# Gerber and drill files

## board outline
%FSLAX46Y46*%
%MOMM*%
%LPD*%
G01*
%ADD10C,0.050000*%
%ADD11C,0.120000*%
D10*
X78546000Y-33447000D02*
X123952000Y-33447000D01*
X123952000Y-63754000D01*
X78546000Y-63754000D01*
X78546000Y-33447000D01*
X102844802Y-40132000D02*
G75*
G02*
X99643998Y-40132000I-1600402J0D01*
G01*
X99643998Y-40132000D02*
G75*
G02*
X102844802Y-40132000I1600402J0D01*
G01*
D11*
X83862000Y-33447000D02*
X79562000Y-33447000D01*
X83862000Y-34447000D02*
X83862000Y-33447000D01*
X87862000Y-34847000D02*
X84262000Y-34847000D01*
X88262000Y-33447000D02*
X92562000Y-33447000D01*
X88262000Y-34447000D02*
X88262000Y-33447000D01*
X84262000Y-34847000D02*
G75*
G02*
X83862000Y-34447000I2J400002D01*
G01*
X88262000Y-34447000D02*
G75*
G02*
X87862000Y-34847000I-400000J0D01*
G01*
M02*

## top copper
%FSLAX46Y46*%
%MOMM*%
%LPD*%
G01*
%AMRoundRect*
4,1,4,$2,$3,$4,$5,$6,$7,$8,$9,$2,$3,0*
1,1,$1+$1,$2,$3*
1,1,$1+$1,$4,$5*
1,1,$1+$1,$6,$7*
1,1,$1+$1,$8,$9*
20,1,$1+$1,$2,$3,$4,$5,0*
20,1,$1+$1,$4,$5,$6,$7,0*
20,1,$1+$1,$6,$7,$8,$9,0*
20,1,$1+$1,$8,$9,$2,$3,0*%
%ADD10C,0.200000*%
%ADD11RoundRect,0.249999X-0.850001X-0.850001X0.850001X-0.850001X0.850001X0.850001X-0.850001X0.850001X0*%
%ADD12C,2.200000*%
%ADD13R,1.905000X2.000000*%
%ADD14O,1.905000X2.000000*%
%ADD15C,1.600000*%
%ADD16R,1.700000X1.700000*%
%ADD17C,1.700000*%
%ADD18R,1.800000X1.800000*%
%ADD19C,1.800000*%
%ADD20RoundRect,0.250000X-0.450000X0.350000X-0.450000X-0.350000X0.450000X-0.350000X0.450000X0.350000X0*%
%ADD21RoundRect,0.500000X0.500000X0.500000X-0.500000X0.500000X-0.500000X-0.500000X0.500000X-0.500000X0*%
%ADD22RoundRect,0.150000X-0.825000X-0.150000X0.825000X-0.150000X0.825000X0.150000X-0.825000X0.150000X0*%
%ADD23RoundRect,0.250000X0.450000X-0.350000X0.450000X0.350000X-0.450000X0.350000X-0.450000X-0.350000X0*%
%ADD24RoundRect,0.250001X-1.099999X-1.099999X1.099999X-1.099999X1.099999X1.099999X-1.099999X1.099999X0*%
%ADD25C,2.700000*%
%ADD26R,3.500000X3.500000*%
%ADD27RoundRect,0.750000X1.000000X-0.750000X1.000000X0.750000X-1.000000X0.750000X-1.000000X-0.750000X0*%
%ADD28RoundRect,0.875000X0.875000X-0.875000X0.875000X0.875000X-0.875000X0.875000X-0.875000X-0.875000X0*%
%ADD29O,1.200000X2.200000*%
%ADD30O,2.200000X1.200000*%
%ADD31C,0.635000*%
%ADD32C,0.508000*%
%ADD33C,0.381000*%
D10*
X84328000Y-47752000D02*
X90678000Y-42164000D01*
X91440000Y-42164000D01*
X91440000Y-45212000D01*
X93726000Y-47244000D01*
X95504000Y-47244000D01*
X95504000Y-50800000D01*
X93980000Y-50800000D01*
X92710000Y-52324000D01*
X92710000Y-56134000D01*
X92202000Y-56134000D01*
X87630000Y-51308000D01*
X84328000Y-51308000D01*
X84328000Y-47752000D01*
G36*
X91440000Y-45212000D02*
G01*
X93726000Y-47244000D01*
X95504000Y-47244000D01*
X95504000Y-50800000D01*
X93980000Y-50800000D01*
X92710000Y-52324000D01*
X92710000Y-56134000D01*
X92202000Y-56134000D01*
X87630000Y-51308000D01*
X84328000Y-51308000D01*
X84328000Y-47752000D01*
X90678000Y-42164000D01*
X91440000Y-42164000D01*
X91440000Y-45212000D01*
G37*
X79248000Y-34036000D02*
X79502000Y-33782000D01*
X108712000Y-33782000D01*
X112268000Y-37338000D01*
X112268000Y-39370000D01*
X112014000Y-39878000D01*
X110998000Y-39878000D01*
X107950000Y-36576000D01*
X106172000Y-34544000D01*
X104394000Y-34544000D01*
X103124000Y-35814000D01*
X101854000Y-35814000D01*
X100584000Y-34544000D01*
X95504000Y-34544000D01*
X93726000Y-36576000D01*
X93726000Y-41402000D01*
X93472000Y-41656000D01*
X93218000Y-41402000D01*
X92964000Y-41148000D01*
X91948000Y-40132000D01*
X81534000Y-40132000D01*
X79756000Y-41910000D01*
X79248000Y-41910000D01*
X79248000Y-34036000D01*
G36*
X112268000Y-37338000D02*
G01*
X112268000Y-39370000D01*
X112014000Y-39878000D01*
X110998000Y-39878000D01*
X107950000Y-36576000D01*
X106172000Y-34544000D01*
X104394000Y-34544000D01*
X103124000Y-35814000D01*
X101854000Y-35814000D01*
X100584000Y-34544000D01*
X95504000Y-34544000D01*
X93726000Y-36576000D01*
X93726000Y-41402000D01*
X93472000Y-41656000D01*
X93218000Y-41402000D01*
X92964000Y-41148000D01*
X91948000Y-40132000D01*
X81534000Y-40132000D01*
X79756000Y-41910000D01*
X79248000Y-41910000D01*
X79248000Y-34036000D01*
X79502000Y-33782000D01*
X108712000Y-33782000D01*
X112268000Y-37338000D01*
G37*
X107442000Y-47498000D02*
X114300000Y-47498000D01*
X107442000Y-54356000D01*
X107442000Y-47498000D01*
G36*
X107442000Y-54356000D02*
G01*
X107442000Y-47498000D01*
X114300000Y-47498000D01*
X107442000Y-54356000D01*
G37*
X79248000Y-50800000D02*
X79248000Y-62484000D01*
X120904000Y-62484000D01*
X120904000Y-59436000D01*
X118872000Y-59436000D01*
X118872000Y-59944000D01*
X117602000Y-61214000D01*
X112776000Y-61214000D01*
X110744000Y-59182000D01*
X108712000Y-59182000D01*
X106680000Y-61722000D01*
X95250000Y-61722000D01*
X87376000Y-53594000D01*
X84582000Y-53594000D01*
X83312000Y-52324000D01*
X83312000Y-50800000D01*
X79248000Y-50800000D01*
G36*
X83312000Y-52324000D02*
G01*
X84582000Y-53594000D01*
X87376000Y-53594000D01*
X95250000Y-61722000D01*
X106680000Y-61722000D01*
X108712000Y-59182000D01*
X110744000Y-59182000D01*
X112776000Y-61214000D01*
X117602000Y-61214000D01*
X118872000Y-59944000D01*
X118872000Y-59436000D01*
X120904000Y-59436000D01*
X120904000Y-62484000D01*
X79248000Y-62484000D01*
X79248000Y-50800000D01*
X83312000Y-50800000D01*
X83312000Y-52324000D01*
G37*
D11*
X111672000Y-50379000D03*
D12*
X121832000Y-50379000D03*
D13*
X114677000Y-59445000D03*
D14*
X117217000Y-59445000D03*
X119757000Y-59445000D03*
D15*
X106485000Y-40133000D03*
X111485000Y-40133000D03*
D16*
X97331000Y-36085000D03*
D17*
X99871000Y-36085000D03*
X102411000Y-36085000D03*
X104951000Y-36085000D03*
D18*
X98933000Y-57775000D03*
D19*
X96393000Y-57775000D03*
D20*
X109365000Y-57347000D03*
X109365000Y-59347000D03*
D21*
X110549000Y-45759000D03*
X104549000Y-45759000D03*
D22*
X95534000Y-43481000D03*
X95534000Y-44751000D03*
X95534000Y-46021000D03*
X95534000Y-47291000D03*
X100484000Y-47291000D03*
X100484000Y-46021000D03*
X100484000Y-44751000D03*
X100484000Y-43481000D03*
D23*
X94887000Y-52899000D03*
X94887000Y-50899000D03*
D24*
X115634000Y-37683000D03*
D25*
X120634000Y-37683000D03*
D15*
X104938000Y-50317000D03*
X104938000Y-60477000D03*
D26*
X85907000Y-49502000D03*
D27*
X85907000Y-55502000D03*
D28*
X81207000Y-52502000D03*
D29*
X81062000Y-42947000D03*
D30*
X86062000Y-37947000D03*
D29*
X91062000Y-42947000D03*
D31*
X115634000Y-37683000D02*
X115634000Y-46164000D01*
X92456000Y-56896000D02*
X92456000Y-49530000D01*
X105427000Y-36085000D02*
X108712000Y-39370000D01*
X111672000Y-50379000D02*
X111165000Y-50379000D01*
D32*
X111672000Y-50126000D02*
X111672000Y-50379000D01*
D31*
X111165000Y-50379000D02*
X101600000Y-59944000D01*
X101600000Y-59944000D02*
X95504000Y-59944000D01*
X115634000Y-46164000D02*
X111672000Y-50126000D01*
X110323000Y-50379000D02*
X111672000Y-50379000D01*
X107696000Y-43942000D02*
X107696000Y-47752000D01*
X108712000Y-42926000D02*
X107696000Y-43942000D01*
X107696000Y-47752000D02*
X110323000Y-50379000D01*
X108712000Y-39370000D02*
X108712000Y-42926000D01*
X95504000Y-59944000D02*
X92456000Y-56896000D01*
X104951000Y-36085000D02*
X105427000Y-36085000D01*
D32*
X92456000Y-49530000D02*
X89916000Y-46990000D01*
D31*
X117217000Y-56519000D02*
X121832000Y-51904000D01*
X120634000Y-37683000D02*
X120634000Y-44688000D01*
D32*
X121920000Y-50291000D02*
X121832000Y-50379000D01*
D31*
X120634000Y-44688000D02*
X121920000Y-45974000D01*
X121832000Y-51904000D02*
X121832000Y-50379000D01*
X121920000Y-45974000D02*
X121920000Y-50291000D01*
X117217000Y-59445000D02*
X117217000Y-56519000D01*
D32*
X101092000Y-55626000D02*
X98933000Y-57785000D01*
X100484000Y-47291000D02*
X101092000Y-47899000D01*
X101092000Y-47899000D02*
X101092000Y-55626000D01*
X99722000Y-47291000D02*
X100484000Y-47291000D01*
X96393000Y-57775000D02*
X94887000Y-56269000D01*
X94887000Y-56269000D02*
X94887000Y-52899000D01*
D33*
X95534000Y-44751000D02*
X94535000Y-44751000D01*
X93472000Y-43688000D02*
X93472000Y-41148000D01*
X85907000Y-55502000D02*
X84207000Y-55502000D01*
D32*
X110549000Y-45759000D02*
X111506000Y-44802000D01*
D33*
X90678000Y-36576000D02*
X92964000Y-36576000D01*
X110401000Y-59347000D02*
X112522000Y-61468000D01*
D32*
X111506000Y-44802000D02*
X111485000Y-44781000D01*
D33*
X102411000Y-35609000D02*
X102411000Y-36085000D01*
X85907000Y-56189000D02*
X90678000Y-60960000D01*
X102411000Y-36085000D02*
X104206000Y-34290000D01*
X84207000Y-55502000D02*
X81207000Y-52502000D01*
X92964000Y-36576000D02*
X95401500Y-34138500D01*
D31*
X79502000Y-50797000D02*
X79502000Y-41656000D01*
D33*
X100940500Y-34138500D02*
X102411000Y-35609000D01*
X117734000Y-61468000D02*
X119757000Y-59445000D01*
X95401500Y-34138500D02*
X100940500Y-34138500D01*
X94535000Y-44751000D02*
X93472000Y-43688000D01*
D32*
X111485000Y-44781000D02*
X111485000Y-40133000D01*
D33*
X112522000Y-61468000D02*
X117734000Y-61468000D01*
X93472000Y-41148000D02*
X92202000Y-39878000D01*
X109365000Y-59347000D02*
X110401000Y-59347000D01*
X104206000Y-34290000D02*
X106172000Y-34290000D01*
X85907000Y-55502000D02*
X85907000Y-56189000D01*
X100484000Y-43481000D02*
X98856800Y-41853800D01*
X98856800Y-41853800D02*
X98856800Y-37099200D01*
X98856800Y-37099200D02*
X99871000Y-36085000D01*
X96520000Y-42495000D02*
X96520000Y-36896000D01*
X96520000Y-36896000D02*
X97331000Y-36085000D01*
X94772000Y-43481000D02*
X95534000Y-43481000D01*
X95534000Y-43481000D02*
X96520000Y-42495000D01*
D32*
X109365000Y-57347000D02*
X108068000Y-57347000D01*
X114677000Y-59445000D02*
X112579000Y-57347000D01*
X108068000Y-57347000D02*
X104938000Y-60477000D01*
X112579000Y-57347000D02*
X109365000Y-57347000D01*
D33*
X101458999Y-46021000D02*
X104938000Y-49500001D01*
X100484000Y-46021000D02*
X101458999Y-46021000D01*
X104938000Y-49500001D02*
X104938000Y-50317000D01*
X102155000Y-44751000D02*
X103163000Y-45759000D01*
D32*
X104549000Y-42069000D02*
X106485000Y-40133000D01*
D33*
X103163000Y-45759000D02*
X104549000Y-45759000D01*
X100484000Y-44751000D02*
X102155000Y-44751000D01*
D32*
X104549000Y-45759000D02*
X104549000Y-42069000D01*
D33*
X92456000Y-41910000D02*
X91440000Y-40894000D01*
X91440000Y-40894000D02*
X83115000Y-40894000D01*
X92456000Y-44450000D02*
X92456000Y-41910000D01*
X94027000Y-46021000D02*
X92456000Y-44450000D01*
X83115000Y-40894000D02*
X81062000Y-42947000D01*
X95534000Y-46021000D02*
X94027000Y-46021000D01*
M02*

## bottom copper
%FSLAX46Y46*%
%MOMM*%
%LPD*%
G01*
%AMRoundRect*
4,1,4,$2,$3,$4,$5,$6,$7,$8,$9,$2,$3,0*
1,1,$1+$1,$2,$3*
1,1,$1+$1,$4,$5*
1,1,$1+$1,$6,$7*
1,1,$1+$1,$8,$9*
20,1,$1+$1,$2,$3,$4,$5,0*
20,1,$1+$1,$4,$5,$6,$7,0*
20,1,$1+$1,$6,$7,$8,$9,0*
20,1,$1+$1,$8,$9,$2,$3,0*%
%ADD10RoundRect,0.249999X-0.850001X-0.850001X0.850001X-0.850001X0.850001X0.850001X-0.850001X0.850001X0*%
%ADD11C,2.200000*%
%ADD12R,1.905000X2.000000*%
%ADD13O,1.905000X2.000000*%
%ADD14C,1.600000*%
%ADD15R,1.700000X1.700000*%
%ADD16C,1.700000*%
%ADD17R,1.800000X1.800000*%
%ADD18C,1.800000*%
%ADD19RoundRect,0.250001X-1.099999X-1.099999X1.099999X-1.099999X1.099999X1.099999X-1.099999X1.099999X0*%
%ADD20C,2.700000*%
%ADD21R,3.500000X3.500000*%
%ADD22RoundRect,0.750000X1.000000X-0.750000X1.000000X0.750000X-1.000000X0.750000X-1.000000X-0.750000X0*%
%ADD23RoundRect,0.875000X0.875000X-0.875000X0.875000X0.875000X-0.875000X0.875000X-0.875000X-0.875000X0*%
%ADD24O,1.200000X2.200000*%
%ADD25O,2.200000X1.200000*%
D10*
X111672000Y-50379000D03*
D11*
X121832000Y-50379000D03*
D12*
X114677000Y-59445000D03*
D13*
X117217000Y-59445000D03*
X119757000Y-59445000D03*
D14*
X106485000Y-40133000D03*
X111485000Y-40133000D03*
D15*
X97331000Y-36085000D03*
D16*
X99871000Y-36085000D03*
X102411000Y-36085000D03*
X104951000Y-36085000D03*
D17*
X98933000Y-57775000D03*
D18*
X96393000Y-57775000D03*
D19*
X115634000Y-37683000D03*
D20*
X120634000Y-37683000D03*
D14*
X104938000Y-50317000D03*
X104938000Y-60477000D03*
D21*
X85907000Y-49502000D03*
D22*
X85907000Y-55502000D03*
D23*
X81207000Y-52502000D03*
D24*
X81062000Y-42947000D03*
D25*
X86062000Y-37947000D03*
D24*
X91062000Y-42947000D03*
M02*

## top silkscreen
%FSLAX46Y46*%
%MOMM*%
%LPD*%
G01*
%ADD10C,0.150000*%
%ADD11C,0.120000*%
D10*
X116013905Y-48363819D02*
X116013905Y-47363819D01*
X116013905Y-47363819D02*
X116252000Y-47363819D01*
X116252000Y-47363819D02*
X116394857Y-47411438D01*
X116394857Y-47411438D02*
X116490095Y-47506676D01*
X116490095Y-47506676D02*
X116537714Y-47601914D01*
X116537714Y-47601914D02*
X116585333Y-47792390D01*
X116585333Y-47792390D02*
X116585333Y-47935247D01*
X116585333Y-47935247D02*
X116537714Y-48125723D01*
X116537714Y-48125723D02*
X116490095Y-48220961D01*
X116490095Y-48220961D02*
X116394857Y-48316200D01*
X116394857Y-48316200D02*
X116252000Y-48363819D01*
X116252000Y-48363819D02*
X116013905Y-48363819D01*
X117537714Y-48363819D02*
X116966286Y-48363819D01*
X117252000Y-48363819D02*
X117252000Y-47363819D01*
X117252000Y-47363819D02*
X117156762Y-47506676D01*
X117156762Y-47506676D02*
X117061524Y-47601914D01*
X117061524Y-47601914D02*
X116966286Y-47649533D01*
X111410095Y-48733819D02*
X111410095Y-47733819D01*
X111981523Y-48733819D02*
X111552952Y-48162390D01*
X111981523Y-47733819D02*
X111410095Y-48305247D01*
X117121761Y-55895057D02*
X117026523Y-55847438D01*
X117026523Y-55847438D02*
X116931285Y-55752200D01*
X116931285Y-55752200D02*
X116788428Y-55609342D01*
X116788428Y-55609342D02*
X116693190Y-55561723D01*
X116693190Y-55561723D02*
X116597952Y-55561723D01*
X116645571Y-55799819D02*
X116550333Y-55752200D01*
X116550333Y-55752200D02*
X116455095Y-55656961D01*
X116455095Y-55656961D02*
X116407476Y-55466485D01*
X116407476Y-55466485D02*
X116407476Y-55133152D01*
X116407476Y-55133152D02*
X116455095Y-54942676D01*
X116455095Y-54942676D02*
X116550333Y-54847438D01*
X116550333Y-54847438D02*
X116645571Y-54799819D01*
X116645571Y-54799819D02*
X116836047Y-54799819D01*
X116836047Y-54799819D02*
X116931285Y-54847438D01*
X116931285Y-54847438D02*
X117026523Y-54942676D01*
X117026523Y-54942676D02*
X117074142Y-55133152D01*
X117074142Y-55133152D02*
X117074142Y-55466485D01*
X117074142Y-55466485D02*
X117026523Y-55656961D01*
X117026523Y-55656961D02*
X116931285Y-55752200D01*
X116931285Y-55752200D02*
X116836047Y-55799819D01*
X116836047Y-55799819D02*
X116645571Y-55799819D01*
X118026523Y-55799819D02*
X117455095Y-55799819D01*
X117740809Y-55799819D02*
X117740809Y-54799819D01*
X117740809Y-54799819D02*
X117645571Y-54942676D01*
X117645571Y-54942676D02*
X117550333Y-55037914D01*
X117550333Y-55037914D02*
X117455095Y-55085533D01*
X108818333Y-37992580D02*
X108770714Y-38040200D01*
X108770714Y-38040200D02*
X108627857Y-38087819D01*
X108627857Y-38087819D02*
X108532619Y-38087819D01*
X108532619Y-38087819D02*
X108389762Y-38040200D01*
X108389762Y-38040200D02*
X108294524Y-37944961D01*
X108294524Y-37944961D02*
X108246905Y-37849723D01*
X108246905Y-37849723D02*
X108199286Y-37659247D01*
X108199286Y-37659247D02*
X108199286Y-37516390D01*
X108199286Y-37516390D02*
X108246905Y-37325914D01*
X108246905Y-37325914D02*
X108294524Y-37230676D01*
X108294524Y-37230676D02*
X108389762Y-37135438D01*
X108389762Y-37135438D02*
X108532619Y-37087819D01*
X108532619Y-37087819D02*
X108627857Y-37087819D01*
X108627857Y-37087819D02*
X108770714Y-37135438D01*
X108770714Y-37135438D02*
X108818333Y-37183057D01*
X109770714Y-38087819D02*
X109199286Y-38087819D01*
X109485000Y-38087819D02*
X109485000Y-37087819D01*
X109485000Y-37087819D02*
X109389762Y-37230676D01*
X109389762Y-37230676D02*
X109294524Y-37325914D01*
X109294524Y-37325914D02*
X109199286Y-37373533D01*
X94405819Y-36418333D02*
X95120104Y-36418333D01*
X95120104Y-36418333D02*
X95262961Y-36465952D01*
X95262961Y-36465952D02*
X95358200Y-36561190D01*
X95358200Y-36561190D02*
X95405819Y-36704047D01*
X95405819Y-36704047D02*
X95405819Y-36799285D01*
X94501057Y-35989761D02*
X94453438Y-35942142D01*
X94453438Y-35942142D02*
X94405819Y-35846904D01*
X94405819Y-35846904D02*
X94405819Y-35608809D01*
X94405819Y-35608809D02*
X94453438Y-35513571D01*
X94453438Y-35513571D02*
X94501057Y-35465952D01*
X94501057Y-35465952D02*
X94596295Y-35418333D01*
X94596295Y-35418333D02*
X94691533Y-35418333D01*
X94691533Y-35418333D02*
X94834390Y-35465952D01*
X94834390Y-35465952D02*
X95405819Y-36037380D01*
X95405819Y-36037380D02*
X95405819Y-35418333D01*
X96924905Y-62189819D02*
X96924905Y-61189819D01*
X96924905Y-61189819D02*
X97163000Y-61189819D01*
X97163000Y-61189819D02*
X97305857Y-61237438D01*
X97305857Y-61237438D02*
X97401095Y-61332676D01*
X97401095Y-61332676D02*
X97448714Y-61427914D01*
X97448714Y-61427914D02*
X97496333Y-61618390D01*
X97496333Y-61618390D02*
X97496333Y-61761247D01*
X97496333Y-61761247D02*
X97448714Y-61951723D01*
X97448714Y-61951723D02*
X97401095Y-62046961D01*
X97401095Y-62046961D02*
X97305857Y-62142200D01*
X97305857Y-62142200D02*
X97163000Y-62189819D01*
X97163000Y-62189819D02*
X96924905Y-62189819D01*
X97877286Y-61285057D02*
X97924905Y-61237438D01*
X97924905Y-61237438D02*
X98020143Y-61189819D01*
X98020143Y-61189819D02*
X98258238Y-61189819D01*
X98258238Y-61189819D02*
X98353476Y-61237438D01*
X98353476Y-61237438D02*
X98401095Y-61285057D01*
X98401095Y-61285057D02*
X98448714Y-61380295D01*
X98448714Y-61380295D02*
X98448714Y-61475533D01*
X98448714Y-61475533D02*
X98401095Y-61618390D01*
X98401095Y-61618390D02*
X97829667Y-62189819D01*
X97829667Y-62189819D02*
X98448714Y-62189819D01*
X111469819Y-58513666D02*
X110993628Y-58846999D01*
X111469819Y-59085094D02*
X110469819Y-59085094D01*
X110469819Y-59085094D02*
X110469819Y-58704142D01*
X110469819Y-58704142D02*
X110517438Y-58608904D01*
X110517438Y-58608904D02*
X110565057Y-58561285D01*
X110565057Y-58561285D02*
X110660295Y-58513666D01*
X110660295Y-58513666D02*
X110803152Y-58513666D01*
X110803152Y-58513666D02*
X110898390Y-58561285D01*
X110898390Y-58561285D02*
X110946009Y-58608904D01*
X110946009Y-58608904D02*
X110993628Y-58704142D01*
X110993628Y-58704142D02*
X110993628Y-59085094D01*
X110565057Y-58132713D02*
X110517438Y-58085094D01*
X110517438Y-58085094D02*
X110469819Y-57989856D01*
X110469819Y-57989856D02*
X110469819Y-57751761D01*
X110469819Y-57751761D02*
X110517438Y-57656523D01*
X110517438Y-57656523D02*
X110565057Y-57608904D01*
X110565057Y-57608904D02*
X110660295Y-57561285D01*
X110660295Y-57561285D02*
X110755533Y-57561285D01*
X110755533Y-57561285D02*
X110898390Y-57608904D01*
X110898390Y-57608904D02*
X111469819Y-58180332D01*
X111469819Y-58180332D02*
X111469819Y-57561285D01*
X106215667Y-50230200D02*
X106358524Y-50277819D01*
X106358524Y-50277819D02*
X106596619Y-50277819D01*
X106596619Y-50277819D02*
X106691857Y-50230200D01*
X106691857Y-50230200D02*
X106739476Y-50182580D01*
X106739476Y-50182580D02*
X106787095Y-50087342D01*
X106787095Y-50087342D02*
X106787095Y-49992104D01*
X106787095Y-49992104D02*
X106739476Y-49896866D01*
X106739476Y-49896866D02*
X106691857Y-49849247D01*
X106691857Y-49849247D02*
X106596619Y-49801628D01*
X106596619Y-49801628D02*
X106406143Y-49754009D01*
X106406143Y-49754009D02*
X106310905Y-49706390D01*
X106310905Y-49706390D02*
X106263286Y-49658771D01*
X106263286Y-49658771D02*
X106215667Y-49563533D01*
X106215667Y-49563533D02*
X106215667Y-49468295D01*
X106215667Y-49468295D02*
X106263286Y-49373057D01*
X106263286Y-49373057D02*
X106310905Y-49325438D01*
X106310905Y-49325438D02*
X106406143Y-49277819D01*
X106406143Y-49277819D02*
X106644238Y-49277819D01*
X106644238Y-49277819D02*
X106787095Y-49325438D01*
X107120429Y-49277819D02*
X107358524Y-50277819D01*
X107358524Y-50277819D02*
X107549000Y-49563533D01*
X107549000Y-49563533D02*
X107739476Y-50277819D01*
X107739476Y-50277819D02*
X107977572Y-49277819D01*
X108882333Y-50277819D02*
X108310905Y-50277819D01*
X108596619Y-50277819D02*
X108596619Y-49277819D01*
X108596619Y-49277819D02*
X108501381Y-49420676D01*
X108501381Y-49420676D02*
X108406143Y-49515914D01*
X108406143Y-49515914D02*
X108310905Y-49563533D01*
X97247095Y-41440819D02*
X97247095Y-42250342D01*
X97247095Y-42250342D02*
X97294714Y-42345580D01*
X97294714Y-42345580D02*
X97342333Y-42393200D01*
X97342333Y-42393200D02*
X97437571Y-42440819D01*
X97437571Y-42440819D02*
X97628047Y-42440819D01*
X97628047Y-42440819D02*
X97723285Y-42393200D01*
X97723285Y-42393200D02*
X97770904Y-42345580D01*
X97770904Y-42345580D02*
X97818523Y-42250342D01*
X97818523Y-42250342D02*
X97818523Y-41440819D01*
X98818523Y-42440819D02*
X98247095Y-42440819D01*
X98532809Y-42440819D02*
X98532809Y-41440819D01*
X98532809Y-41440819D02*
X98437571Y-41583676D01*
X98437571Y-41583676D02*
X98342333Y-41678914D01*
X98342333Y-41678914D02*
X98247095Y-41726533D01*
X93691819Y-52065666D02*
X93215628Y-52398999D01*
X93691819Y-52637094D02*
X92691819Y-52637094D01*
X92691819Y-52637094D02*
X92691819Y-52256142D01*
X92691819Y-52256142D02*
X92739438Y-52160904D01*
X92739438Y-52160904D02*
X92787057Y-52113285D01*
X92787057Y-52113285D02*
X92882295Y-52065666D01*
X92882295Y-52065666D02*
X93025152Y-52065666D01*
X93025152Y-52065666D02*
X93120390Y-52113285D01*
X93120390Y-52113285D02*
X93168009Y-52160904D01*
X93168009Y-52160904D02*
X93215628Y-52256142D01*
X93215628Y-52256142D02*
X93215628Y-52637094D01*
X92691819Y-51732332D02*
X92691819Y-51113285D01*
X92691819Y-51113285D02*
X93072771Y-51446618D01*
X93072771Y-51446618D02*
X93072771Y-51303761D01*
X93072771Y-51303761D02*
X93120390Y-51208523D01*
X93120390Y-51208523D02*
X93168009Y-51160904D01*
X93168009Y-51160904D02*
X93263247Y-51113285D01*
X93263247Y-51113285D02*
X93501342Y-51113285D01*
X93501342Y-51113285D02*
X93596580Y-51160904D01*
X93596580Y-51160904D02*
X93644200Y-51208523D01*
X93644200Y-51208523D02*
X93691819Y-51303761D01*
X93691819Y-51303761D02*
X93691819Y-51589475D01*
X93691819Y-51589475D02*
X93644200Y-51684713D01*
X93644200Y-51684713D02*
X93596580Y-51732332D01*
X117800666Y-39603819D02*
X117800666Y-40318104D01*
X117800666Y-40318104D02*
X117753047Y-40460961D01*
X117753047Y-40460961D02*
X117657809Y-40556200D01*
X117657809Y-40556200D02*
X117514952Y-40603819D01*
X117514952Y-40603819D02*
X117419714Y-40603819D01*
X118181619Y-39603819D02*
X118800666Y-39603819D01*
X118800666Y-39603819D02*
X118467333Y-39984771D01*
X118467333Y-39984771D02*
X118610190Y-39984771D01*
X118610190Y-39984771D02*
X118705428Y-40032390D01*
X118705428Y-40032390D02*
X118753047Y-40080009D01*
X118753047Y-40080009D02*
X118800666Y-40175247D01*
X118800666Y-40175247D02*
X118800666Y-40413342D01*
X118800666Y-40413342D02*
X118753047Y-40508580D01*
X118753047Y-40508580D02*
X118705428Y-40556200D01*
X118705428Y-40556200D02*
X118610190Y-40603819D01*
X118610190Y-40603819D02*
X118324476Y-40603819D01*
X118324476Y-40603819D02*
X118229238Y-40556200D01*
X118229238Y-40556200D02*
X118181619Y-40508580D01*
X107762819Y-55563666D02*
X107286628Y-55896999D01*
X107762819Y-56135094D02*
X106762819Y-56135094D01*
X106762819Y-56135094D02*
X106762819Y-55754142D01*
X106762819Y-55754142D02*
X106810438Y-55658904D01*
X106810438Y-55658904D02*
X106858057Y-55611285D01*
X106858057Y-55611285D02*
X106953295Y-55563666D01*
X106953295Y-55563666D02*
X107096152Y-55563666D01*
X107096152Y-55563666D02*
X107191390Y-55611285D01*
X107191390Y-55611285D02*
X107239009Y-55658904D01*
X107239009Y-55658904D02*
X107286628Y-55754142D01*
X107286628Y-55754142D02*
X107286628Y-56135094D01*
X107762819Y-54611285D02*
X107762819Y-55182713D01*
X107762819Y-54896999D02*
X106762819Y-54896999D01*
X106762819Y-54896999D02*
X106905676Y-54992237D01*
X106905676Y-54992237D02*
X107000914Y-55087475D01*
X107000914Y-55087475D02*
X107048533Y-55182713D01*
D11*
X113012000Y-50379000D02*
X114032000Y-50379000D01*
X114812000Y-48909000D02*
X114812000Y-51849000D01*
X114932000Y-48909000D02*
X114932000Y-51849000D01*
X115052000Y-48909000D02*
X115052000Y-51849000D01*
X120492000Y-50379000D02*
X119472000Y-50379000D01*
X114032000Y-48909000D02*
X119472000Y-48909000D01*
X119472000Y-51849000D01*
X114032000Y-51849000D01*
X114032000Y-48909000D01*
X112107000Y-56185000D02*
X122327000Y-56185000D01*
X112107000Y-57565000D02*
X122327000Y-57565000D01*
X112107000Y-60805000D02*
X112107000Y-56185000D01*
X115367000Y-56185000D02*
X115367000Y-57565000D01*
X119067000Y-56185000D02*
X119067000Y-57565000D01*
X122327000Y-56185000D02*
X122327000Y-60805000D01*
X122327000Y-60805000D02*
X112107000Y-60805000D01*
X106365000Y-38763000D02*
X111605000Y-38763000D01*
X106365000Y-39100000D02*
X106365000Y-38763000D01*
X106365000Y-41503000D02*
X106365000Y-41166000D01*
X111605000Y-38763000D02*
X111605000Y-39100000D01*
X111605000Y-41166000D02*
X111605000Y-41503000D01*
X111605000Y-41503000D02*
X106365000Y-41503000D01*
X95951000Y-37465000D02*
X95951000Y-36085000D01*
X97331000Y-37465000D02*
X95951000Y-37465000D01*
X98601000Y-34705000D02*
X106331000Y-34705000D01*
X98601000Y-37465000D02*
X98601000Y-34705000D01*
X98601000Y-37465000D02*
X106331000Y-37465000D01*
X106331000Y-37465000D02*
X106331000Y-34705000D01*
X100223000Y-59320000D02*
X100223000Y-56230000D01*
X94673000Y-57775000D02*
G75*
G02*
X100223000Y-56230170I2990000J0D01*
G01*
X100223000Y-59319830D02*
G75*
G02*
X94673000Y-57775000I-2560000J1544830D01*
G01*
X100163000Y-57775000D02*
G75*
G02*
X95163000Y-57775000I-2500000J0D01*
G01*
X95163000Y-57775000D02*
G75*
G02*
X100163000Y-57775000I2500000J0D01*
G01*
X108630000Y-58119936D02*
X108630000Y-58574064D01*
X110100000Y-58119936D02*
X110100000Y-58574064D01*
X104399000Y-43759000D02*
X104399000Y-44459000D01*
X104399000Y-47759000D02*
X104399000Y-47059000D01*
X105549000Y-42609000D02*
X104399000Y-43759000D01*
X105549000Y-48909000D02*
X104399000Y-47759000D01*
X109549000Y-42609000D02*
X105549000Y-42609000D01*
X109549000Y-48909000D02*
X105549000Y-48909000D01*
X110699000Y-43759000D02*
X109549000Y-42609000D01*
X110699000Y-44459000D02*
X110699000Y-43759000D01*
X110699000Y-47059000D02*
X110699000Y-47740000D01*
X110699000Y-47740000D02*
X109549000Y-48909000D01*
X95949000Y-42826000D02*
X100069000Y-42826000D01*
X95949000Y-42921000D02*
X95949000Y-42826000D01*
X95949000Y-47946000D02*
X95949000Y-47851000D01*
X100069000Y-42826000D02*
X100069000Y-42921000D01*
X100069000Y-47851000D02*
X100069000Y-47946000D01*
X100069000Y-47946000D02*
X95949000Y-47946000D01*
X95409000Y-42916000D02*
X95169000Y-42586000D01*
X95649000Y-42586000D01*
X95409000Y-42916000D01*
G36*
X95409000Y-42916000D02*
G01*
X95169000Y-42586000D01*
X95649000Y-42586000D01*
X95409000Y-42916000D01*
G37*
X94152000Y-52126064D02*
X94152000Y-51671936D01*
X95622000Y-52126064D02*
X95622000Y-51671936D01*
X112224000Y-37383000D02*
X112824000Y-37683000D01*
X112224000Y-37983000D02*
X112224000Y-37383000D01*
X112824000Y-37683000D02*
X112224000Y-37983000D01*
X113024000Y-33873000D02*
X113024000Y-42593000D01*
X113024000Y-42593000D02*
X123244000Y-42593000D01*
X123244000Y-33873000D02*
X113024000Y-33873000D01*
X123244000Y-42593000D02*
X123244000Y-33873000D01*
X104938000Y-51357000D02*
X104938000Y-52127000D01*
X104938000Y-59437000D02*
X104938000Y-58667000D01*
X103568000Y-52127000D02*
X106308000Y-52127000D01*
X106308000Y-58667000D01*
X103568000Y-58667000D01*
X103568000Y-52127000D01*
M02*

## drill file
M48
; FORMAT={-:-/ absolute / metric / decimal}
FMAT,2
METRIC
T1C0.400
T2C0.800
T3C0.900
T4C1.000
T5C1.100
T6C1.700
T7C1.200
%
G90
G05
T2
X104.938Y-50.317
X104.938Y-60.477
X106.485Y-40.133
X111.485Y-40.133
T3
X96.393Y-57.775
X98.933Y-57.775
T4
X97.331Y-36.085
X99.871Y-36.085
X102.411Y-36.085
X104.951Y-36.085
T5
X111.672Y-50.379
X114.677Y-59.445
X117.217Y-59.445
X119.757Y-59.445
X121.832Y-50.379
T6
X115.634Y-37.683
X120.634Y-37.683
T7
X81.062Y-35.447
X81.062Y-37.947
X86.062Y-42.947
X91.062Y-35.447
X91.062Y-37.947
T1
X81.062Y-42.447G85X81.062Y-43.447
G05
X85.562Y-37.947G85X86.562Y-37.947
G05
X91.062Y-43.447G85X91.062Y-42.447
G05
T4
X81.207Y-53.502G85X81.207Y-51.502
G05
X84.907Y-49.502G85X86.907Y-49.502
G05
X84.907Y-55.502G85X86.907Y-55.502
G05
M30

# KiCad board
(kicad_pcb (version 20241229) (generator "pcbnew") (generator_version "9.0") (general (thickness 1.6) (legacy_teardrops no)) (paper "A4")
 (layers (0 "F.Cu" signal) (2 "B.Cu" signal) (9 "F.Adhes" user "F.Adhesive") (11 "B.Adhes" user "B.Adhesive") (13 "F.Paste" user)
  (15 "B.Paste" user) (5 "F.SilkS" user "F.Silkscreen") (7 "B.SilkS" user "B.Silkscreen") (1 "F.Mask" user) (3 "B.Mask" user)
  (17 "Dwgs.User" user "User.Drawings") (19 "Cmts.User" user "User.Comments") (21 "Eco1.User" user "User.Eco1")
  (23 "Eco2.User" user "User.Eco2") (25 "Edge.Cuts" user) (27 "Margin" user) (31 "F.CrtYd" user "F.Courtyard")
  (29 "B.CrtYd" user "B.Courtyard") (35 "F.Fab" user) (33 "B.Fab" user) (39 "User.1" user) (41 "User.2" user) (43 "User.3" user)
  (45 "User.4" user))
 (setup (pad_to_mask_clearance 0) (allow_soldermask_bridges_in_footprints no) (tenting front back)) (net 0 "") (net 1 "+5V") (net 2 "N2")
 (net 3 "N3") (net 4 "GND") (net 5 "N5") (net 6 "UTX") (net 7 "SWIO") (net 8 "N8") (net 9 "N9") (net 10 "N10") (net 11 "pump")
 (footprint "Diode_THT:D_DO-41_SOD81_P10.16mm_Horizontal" (layer "F.Cu") (at 111.672 50.379)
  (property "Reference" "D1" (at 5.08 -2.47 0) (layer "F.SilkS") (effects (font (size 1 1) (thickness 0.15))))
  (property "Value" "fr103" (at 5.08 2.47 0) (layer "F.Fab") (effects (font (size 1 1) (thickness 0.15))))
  (fp_line (start 1.34 0) (end 2.36 0) (stroke (width 0.12) (type solid)) (layer "F.SilkS"))
  (fp_line (start 3.14 -1.47) (end 3.14 1.47) (stroke (width 0.12) (type solid)) (layer "F.SilkS"))
  (fp_line (start 3.26 -1.47) (end 3.26 1.47) (stroke (width 0.12) (type solid)) (layer "F.SilkS"))
  (fp_line (start 3.38 -1.47) (end 3.38 1.47) (stroke (width 0.12) (type solid)) (layer "F.SilkS"))
  (fp_line (start 8.82 0) (end 7.8 0) (stroke (width 0.12) (type solid)) (layer "F.SilkS"))
  (fp_rect (start 2.36 -1.47) (end 7.8 1.47) (stroke (width 0.12) (type solid)) (fill no) (layer "F.SilkS"))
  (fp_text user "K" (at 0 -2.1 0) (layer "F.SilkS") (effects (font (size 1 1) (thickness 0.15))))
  (pad "1" thru_hole roundrect (at 0 0) (size 2.2 2.2) (drill 1.1) (layers "*.Cu" "*.Mask") (remove_unused_layers no)
   (roundrect_rratio 0.113636) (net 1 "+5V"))
  (pad "2" thru_hole circle (at 10.16 0) (size 2.2 2.2) (drill 1.1) (layers "*.Cu" "*.Mask") (remove_unused_layers no) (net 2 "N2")))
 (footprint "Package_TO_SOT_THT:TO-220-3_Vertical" (layer "F.Cu") (at 114.677 59.445)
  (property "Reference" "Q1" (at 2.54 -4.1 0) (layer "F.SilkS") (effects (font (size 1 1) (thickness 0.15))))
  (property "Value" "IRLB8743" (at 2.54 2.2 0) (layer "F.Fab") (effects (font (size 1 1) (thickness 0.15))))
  (fp_line (start -2.57 -3.26) (end 7.65 -3.26) (stroke (width 0.12) (type solid)) (layer "F.SilkS"))
  (fp_line (start -2.57 -1.88) (end 7.65 -1.88) (stroke (width 0.12) (type solid)) (layer "F.SilkS"))
  (fp_line (start -2.57 1.36) (end -2.57 -3.26) (stroke (width 0.12) (type solid)) (layer "F.SilkS"))
  (fp_line (start 0.69 -3.26) (end 0.69 -1.88) (stroke (width 0.12) (type solid)) (layer "F.SilkS"))
  (fp_line (start 4.39 -3.26) (end 4.39 -1.88) (stroke (width 0.12) (type solid)) (layer "F.SilkS"))
  (fp_line (start 7.65 -3.26) (end 7.65 1.36) (stroke (width 0.12) (type solid)) (layer "F.SilkS"))
  (fp_line (start 7.65 1.36) (end -2.57 1.36) (stroke (width 0.12) (type solid)) (layer "F.SilkS"))
  (pad "1" thru_hole rect (at 0 0) (size 1.905 2) (drill 1.1) (layers "*.Cu" "*.Mask") (remove_unused_layers no) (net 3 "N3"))
  (pad "2" thru_hole oval (at 2.54 0) (size 1.905 2) (drill 1.1) (layers "*.Cu" "*.Mask") (remove_unused_layers no) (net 2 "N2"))
  (pad "3" thru_hole oval (at 5.08 0) (size 1.905 2) (drill 1.1) (layers "*.Cu" "*.Mask") (remove_unused_layers no) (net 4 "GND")))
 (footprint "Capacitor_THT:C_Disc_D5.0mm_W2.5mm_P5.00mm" (layer "F.Cu") (at 106.485 40.133)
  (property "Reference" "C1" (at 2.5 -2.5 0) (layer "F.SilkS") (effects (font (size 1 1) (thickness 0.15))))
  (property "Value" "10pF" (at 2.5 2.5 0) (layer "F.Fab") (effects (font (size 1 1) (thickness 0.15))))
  (fp_line (start -0.12 -1.37) (end 5.12 -1.37) (stroke (width 0.12) (type solid)) (layer "F.SilkS"))
  (fp_line (start -0.12 -1.033) (end -0.12 -1.37) (stroke (width 0.12) (type solid)) (layer "F.SilkS"))
  (fp_line (start -0.12 1.37) (end -0.12 1.033) (stroke (width 0.12) (type solid)) (layer "F.SilkS"))
  (fp_line (start 5.12 -1.37) (end 5.12 -1.033) (stroke (width 0.12) (type solid)) (layer "F.SilkS"))
  (fp_line (start 5.12 1.033) (end 5.12 1.37) (stroke (width 0.12) (type solid)) (layer "F.SilkS"))
  (fp_line (start 5.12 1.37) (end -0.12 1.37) (stroke (width 0.12) (type solid)) (layer "F.SilkS"))
  (pad "1" thru_hole circle (at 0 0) (size 1.6 1.6) (drill 0.8) (layers "*.Cu" "*.Mask") (remove_unused_layers no) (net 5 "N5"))
  (pad "2" thru_hole circle (at 5 0) (size 1.6 1.6) (drill 0.8) (layers "*.Cu" "*.Mask") (remove_unused_layers no) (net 4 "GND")))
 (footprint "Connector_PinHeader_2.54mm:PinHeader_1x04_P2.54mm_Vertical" (layer "F.Cu") (at 97.331 36.085 90)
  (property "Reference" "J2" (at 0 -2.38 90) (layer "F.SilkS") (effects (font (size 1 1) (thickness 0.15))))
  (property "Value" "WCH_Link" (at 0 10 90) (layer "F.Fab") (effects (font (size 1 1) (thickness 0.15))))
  (fp_line (start -1.38 -1.38) (end 0 -1.38) (stroke (width 0.12) (type solid)) (layer "F.SilkS"))
  (fp_line (start -1.38 0) (end -1.38 -1.38) (stroke (width 0.12) (type solid)) (layer "F.SilkS"))
  (fp_line (start 1.38 1.27) (end 1.38 9) (stroke (width 0.12) (type solid)) (layer "F.SilkS"))
  (fp_line (start -1.38 1.27) (end 1.38 1.27) (stroke (width 0.12) (type solid)) (layer "F.SilkS"))
  (fp_line (start -1.38 1.27) (end -1.38 9) (stroke (width 0.12) (type solid)) (layer "F.SilkS"))
  (fp_line (start -1.38 9) (end 1.38 9) (stroke (width 0.12) (type solid)) (layer "F.SilkS"))
  (pad "1" thru_hole rect (at 0 0 90) (size 1.7 1.7) (drill 1) (layers "*.Cu" "*.Mask") (remove_unused_layers no) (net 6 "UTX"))
  (pad "2" thru_hole circle (at 0 2.54 90) (size 1.7 1.7) (drill 1) (layers "*.Cu" "*.Mask") (remove_unused_layers no) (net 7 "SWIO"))
  (pad "3" thru_hole circle (at 0 5.08 90) (size 1.7 1.7) (drill 1) (layers "*.Cu" "*.Mask") (remove_unused_layers no) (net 4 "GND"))
  (pad "4" thru_hole circle (at 0 7.62 90) (size 1.7 1.7) (drill 1) (layers "*.Cu" "*.Mask") (remove_unused_layers no) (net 1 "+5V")))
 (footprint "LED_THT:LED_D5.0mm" (layer "F.Cu") (at 98.933 57.775 180)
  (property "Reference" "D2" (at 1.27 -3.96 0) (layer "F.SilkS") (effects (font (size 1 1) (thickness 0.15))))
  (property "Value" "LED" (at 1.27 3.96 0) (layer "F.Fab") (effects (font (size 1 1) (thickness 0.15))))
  (fp_line (start -1.29 -1.545) (end -1.29 1.545) (stroke (width 0.12) (type solid)) (layer "F.SilkS"))
  (fp_arc (start 4.26 0) (mid 2.071779 2.880495) (end -1.29 1.54483) (stroke (width 0.12) (type solid)) (layer "F.SilkS"))
  (fp_arc (start -1.29 -1.54483) (mid 2.071779 -2.880495) (end 4.26 0) (stroke (width 0.12) (type solid)) (layer "F.SilkS"))
  (fp_circle (center 1.27 0) (end 3.77 0) (stroke (width 0.12) (type solid)) (fill no) (layer "F.SilkS"))
  (pad "1" thru_hole rect (at 0 0 180) (size 1.8 1.8) (drill 0.9) (layers "*.Cu" "*.Mask") (remove_unused_layers no) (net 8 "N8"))
  (pad "2" thru_hole circle (at 2.54 0 180) (size 1.8 1.8) (drill 0.9) (layers "*.Cu" "*.Mask") (remove_unused_layers no) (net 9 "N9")))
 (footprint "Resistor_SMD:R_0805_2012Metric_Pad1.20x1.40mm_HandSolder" (layer "F.Cu") (at 109.365 58.347 -90)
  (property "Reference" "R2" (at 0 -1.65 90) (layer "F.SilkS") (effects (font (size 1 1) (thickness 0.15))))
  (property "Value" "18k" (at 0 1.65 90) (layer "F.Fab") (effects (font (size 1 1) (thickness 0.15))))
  (fp_line (start -0.227064 0.735) (end 0.227064 0.735) (stroke (width 0.12) (type solid)) (layer "F.SilkS"))
  (fp_line (start -0.227064 -0.735) (end 0.227064 -0.735) (stroke (width 0.12) (type solid)) (layer "F.SilkS"))
  (pad "1" smd roundrect (at -1 0 270) (size 1.2 1.4) (layers "F.Cu" "F.Mask" "F.Paste") (roundrect_rratio 0.208333) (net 3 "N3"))
  (pad "2" smd roundrect (at 1 0 270) (size 1.2 1.4) (layers "F.Cu" "F.Mask" "F.Paste") (roundrect_rratio 0.208333) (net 4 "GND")))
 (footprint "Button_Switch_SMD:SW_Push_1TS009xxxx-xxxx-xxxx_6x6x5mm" (layer "F.Cu") (at 107.549 45.759 180)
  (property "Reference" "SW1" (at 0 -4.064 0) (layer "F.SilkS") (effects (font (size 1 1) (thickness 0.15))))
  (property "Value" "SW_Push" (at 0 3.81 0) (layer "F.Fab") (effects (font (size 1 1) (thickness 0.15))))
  (fp_line (start 3.15 2) (end 3.15 1.3) (stroke (width 0.12) (type default)) (layer "F.SilkS"))
  (fp_line (start 3.15 -2) (end 3.15 -1.3) (stroke (width 0.12) (type default)) (layer "F.SilkS"))
  (fp_line (start 2 3.15) (end 3.15 2) (stroke (width 0.12) (type default)) (layer "F.SilkS"))
  (fp_line (start 2 -3.15) (end 3.15 -2) (stroke (width 0.12) (type default)) (layer "F.SilkS"))
  (fp_line (start -2 3.15) (end 2 3.15) (stroke (width 0.12) (type default)) (layer "F.SilkS"))
  (fp_line (start -2 -3.15) (end 2 -3.15) (stroke (width 0.12) (type default)) (layer "F.SilkS"))
  (fp_line (start -3.15 2) (end -2 3.15) (stroke (width 0.12) (type default)) (layer "F.SilkS"))
  (fp_line (start -3.15 1.3) (end -3.15 2) (stroke (width 0.12) (type default)) (layer "F.SilkS"))
  (fp_line (start -3.15 -1.3) (end -3.15 -1.981) (stroke (width 0.12) (type default)) (layer "F.SilkS"))
  (fp_line (start -3.15 -1.981) (end -2 -3.15) (stroke (width 0.12) (type default)) (layer "F.SilkS"))
  (pad "1" smd roundrect (at -3 0 180) (size 2 2) (layers "F.Cu" "F.Mask" "F.Paste") (roundrect_rratio 0.25) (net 4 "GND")
   (thermal_bridge_angle 45))
  (pad "2" smd roundrect (at 3 0 180) (size 2 2) (layers "F.Cu" "F.Mask" "F.Paste") (roundrect_rratio 0.25) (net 5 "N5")
   (thermal_bridge_angle 45)))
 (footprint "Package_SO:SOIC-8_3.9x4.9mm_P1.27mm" (layer "F.Cu") (at 98.009 45.386)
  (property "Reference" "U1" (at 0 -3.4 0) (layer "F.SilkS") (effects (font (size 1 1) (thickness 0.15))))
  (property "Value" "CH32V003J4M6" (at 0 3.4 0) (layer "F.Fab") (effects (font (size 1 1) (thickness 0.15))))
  (fp_line (start -2.06 -2.56) (end 2.06 -2.56) (stroke (width 0.12) (type solid)) (layer "F.SilkS"))
  (fp_line (start -2.06 -2.465) (end -2.06 -2.56) (stroke (width 0.12) (type solid)) (layer "F.SilkS"))
  (fp_line (start -2.06 2.56) (end -2.06 2.465) (stroke (width 0.12) (type solid)) (layer "F.SilkS"))
  (fp_line (start 2.06 -2.56) (end 2.06 -2.465) (stroke (width 0.12) (type solid)) (layer "F.SilkS"))
  (fp_line (start 2.06 2.465) (end 2.06 2.56) (stroke (width 0.12) (type solid)) (layer "F.SilkS"))
  (fp_line (start 2.06 2.56) (end -2.06 2.56) (stroke (width 0.12) (type solid)) (layer "F.SilkS"))
  (fp_poly (pts (xy -2.6 -2.47) (xy -2.84 -2.8) (xy -2.36 -2.8)) (stroke (width 0.12) (type solid)) (fill yes) (layer "F.SilkS"))
  (pad "1" smd roundrect (at -2.475 -1.905) (size 1.95 0.6) (layers "F.Cu" "F.Mask" "F.Paste") (roundrect_rratio 0.25) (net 6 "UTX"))
  (pad "2" smd roundrect (at -2.475 -0.635) (size 1.95 0.6) (layers "F.Cu" "F.Mask" "F.Paste") (roundrect_rratio 0.25) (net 4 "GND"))
  (pad "3" smd roundrect (at -2.475 0.635) (size 1.95 0.6) (layers "F.Cu" "F.Mask" "F.Paste") (roundrect_rratio 0.25) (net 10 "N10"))
  (pad "4" smd roundrect (at -2.475 1.905) (size 1.95 0.6) (layers "F.Cu" "F.Mask" "F.Paste") (roundrect_rratio 0.25) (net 1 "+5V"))
  (pad "5" smd roundrect (at 2.475 1.905) (size 1.95 0.6) (layers "F.Cu" "F.Mask" "F.Paste") (roundrect_rratio 0.25) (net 8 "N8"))
  (pad "6" smd roundrect (at 2.475 0.635) (size 1.95 0.6) (layers "F.Cu" "F.Mask" "F.Paste") (roundrect_rratio 0.25) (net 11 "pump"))
  (pad "7" smd roundrect (at 2.475 -0.635) (size 1.95 0.6) (layers "F.Cu" "F.Mask" "F.Paste") (roundrect_rratio 0.25) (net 5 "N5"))
  (pad "8" smd roundrect (at 2.475 -1.905) (size 1.95 0.6) (layers "F.Cu" "F.Mask" "F.Paste") (roundrect_rratio 0.25) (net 7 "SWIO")))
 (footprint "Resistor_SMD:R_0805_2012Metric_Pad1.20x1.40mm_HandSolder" (layer "F.Cu") (at 94.887 51.899 90)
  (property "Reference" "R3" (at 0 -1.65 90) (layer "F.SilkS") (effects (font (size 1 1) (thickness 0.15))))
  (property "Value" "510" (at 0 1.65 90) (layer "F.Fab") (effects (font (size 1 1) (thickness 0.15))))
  (fp_line (start -0.227064 -0.735) (end 0.227064 -0.735) (stroke (width 0.12) (type solid)) (layer "F.SilkS"))
  (fp_line (start -0.227064 0.735) (end 0.227064 0.735) (stroke (width 0.12) (type solid)) (layer "F.SilkS"))
  (pad "1" smd roundrect (at -1 0 90) (size 1.2 1.4) (layers "F.Cu" "F.Mask" "F.Paste") (roundrect_rratio 0.208333) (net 9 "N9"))
  (pad "2" smd roundrect (at 1 0 90) (size 1.2 1.4) (layers "F.Cu" "F.Mask" "F.Paste") (roundrect_rratio 0.208333) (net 1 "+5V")))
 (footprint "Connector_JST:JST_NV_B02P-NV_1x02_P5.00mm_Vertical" (layer "F.Cu") (at 115.634 37.683)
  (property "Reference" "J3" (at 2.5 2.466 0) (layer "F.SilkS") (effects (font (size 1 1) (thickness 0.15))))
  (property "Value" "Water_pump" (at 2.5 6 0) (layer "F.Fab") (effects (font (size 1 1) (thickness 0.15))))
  (fp_line (start -3.41 -0.3) (end -2.81 0) (stroke (width 0.12) (type solid)) (layer "F.SilkS"))
  (fp_line (start -3.41 0.3) (end -3.41 -0.3) (stroke (width 0.12) (type solid)) (layer "F.SilkS"))
  (fp_line (start -2.81 0) (end -3.41 0.3) (stroke (width 0.12) (type solid)) (layer "F.SilkS"))
  (fp_line (start -2.61 -3.81) (end -2.61 4.91) (stroke (width 0.12) (type solid)) (layer "F.SilkS"))
  (fp_line (start -2.61 4.91) (end 7.61 4.91) (stroke (width 0.12) (type solid)) (layer "F.SilkS"))
  (fp_line (start 7.61 -3.81) (end -2.61 -3.81) (stroke (width 0.12) (type solid)) (layer "F.SilkS"))
  (fp_line (start 7.61 4.91) (end 7.61 -3.81) (stroke (width 0.12) (type solid)) (layer "F.SilkS"))
  (pad "1" thru_hole roundrect (at 0 0) (size 2.7 2.7) (drill 1.7) (layers "*.Cu" "*.Mask") (remove_unused_layers no)
   (roundrect_rratio 0.092593) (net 1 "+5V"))
  (pad "2" thru_hole circle (at 5 0) (size 2.7 2.7) (drill 1.7) (layers "*.Cu" "*.Mask") (remove_unused_layers no) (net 2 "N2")))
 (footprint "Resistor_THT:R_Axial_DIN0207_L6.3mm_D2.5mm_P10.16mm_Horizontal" (layer "F.Cu") (at 104.938 50.317 -90)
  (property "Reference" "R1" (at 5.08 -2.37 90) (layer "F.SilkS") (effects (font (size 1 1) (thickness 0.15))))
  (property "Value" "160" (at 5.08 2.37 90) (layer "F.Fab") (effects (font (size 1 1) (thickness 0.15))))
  (fp_line (start 1.04 0) (end 1.81 0) (stroke (width 0.12) (type solid)) (layer "F.SilkS"))
  (fp_line (start 9.12 0) (end 8.35 0) (stroke (width 0.12) (type solid)) (layer "F.SilkS"))
  (fp_rect (start 1.81 -1.37) (end 8.35 1.37) (stroke (width 0.12) (type solid)) (fill no) (layer "F.SilkS"))
  (pad "1" thru_hole circle (at 0 0 270) (size 1.6 1.6) (drill 0.8) (layers "*.Cu" "*.Mask") (remove_unused_layers no) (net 11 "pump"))
  (pad "2" thru_hole circle (at 10.16 0 270) (size 1.6 1.6) (drill 0.8) (layers "*.Cu" "*.Mask") (remove_unused_layers no) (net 3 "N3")))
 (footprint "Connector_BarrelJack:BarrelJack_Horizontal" (layer "B.Cu") (at 85.907 49.502 90)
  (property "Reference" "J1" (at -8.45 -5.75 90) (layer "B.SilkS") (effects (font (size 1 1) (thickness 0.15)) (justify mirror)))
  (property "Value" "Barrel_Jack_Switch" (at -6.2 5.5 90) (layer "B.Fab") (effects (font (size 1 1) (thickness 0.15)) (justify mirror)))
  (pad "1" thru_hole rect (at 0 0 90) (size 3.5 3.5) (drill oval 1 3) (layers "*.Cu" "*.Mask") (remove_unused_layers no) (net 1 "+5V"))
  (pad "2" thru_hole roundrect (at -6 0 90) (size 3 3.5) (drill oval 1 3) (layers "*.Cu" "*.Mask") (remove_unused_layers no)
   (roundrect_rratio 0.25) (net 4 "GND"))
  (pad "3" thru_hole roundrect (at -3 -4.7 90) (size 3.5 3.5) (drill oval 3 1) (layers "*.Cu" "*.Mask") (remove_unused_layers no)
   (roundrect_rratio 0.25) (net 4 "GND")))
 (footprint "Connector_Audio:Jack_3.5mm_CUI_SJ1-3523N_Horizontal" (layer "B.Cu") (at 86.062 37.947)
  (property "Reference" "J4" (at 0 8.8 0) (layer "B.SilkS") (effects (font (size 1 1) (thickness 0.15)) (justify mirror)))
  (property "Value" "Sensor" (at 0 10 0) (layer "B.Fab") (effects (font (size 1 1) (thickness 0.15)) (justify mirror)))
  (fp_line (start -2.2 -4.5) (end -6.5 -4.5) (stroke (width 0.12) (type solid)) (layer "Edge.Cuts"))
  (fp_line (start -2.2 -3.5) (end -2.2 -4.5) (stroke (width 0.12) (type solid)) (layer "Edge.Cuts"))
  (fp_line (start 1.8 -3.1) (end -1.8 -3.1) (stroke (width 0.12) (type solid)) (layer "Edge.Cuts"))
  (fp_line (start 2.2 -4.5) (end 6.5 -4.5) (stroke (width 0.12) (type solid)) (layer "Edge.Cuts"))
  (fp_line (start 2.2 -3.5) (end 2.2 -4.5) (stroke (width 0.12) (type solid)) (layer "Edge.Cuts"))
  (fp_arc (start -1.8 -3.1) (mid -2.082842 -3.217158) (end -2.2 -3.5) (stroke (width 0.12) (type solid)) (layer "Edge.Cuts"))
  (fp_arc (start 2.2 -3.5) (mid 2.082843 -3.217157) (end 1.8 -3.1) (stroke (width 0.12) (type solid)) (layer "Edge.Cuts"))
  (pad "" np_thru_hole circle (at -5 -2.5) (size 1.2 1.2) (drill 1.2) (layers "*.Cu" "*.Mask"))
  (pad "" np_thru_hole circle (at -5 0) (size 1.2 1.2) (drill 1.2) (layers "*.Cu" "*.Mask"))
  (pad "" np_thru_hole circle (at 0 5) (size 1.2 1.2) (drill 1.2) (layers "*.Cu" "*.Mask"))
  (pad "" np_thru_hole circle (at 5 -2.5) (size 1.2 1.2) (drill 1.2) (layers "*.Cu" "*.Mask"))
  (pad "" np_thru_hole circle (at 5 0) (size 1.2 1.2) (drill 1.2) (layers "*.Cu" "*.Mask"))
  (pad "R" thru_hole oval (at -5 5) (size 1.2 2.2) (drill oval 0.4 1.4) (layers "*.Cu" "*.Mask") (remove_unused_layers no) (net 10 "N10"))
  (pad "S" thru_hole oval (at 0 0) (size 2.2 1.2) (drill oval 1.4 0.4) (layers "*.Cu" "*.Mask") (remove_unused_layers no) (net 4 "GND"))
  (pad "T" thru_hole oval (at 5 5 180) (size 1.2 2.2) (drill oval 0.4 1.4) (layers "*.Cu" "*.Mask") (remove_unused_layers no) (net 1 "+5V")))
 (gr_poly
  (pts (xy 84.328 47.752) (xy 90.678 42.164) (xy 91.44 42.164) (xy 91.44 45.212) (xy 93.726 47.244) (xy 95.504 47.244) (xy 95.504 50.8)
   (xy 93.98 50.8) (xy 92.71 52.324) (xy 92.71 56.134) (xy 92.202 56.134) (xy 87.63 51.308) (xy 84.328 51.308))
  (stroke (width 0.2) (type solid)) (fill yes) (layer "F.Cu") (net 1))
 (gr_poly
  (pts (xy 79.248 34.036) (xy 79.502 33.782) (xy 108.712 33.782) (xy 112.268 37.338) (xy 112.268 39.37) (xy 112.014 39.878)
   (xy 110.998 39.878) (xy 107.95 36.576) (xy 106.172 34.544) (xy 104.394 34.544) (xy 103.124 35.814) (xy 101.854 35.814)
   (xy 100.584 34.544) (xy 95.504 34.544) (xy 93.726 36.576) (xy 93.726 41.402) (xy 93.472 41.656) (xy 93.218 41.402) (xy 92.964 41.148)
   (xy 91.948 40.132) (xy 81.534 40.132) (xy 79.756 41.91) (xy 79.248 41.91))
  (stroke (width 0.2) (type solid)) (fill yes) (layer "F.Cu") (net 4))
 (gr_poly
  (pts (xy 107.442 47.498) (xy 114.3 47.498) (xy 107.442 54.356)) (stroke (width 0.2) (type solid)) (fill yes) (layer "F.Cu") (net 1))
 (gr_poly
  (pts (xy 79.248 50.8) (xy 79.248 62.484) (xy 120.904 62.484) (xy 120.904 59.436) (xy 118.872 59.436) (xy 118.872 59.944)
   (xy 117.602 61.214) (xy 112.776 61.214) (xy 110.744 59.182) (xy 108.712 59.182) (xy 106.68 61.722) (xy 95.25 61.722) (xy 87.376 53.594)
   (xy 84.582 53.594) (xy 83.312 52.324) (xy 83.312 50.8))
  (stroke (width 0.2) (type solid)) (fill yes) (layer "F.Cu") (net 4))
 (gr_rect (start 78.546 33.447) (end 123.952 63.754) (stroke (width 0.05) (type default)) (fill no) (layer "Edge.Cuts"))
 (gr_circle (center 101.2444 40.132) (end 102.8446 40.1574) (stroke (width 0.05) (type default)) (fill no) (layer "Edge.Cuts"))
 (segment (start 115.634 37.683) (end 115.634 46.164) (width 0.635) (layer "F.Cu") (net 1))
 (segment (start 92.456 56.896) (end 92.456 49.53) (width 0.635) (layer "F.Cu") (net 1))
 (segment (start 105.427 36.085) (end 108.712 39.37) (width 0.635) (layer "F.Cu") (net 1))
 (segment (start 111.672 50.379) (end 111.165 50.379) (width 0.635) (layer "F.Cu") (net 1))
 (segment (start 111.672 50.126) (end 111.672 50.379) (width 0.508) (layer "F.Cu") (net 1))
 (segment (start 111.165 50.379) (end 101.6 59.944) (width 0.635) (layer "F.Cu") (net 1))
 (segment (start 101.6 59.944) (end 95.504 59.944) (width 0.635) (layer "F.Cu") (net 1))
 (segment (start 115.634 46.164) (end 111.672 50.126) (width 0.635) (layer "F.Cu") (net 1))
 (segment (start 110.323 50.379) (end 111.672 50.379) (width 0.635) (layer "F.Cu") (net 1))
 (segment (start 107.696 43.942) (end 107.696 47.752) (width 0.635) (layer "F.Cu") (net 1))
 (segment (start 108.712 42.926) (end 107.696 43.942) (width 0.635) (layer "F.Cu") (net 1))
 (segment (start 107.696 47.752) (end 110.323 50.379) (width 0.635) (layer "F.Cu") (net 1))
 (segment (start 108.712 39.37) (end 108.712 42.926) (width 0.635) (layer "F.Cu") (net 1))
 (segment (start 95.504 59.944) (end 92.456 56.896) (width 0.635) (layer "F.Cu") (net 1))
 (segment (start 104.951 36.085) (end 105.427 36.085) (width 0.635) (layer "F.Cu") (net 1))
 (segment (start 92.456 49.53) (end 89.916 46.99) (width 0.508) (layer "F.Cu") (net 1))
 (segment (start 117.217 56.519) (end 121.832 51.904) (width 0.635) (layer "F.Cu") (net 2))
 (segment (start 120.634 37.683) (end 120.634 44.688) (width 0.635) (layer "F.Cu") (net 2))
 (segment (start 121.92 50.291) (end 121.832 50.379) (width 0.508) (layer "F.Cu") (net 2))
 (segment (start 120.634 44.688) (end 121.92 45.974) (width 0.635) (layer "F.Cu") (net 2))
 (segment (start 121.832 51.904) (end 121.832 50.379) (width 0.635) (layer "F.Cu") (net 2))
 (segment (start 121.92 45.974) (end 121.92 50.291) (width 0.635) (layer "F.Cu") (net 2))
 (segment (start 117.217 59.445) (end 117.217 56.519) (width 0.635) (layer "F.Cu") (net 2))
 (segment (start 101.092 55.626) (end 98.933 57.785) (width 0.508) (layer "F.Cu") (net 8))
 (segment (start 100.484 47.291) (end 101.092 47.899) (width 0.508) (layer "F.Cu") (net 8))
 (segment (start 101.092 47.899) (end 101.092 55.626) (width 0.508) (layer "F.Cu") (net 8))
 (segment (start 99.722 47.291) (end 100.484 47.291) (width 0.508) (layer "F.Cu") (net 8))
 (segment (start 96.393 57.775) (end 94.887 56.269) (width 0.508) (layer "F.Cu") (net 9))
 (segment (start 94.887 56.269) (end 94.887 52.899) (width 0.508) (layer "F.Cu") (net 9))
 (segment (start 95.534 44.751) (end 94.535 44.751) (width 0.381) (layer "F.Cu") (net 4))
 (segment (start 93.472 43.688) (end 93.472 41.148) (width 0.381) (layer "F.Cu") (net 4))
 (segment (start 85.907 55.502) (end 84.207 55.502) (width 0.381) (layer "F.Cu") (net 4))
 (segment (start 110.549 45.759) (end 111.506 44.802) (width 0.508) (layer "F.Cu") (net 4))
 (segment (start 90.678 36.576) (end 92.964 36.576) (width 0.381) (layer "F.Cu") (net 4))
 (segment (start 110.401 59.347) (end 112.522 61.468) (width 0.381) (layer "F.Cu") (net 4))
 (segment (start 111.506 44.802) (end 111.485 44.781) (width 0.508) (layer "F.Cu") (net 4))
 (segment (start 102.411 35.609) (end 102.411 36.085) (width 0.381) (layer "F.Cu") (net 4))
 (segment (start 85.907 56.189) (end 90.678 60.96) (width 0.381) (layer "F.Cu") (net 4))
 (segment (start 102.411 36.085) (end 104.206 34.29) (width 0.381) (layer "F.Cu") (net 4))
 (segment (start 84.207 55.502) (end 81.207 52.502) (width 0.381) (layer "F.Cu") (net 4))
 (segment (start 92.964 36.576) (end 95.4015 34.1385) (width 0.381) (layer "F.Cu") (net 4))
 (segment (start 79.502 50.797) (end 79.502 41.656) (width 0.635) (layer "F.Cu") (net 4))
 (segment (start 100.9405 34.1385) (end 102.411 35.609) (width 0.381) (layer "F.Cu") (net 4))
 (segment (start 117.734 61.468) (end 119.757 59.445) (width 0.381) (layer "F.Cu") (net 4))
 (segment (start 95.4015 34.1385) (end 100.9405 34.1385) (width 0.381) (layer "F.Cu") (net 4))
 (segment (start 94.535 44.751) (end 93.472 43.688) (width 0.381) (layer "F.Cu") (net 4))
 (segment (start 111.485 44.781) (end 111.485 40.133) (width 0.508) (layer "F.Cu") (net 4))
 (segment (start 112.522 61.468) (end 117.734 61.468) (width 0.381) (layer "F.Cu") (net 4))
 (segment (start 93.472 41.148) (end 92.202 39.878) (width 0.381) (layer "F.Cu") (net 4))
 (segment (start 109.365 59.347) (end 110.401 59.347) (width 0.381) (layer "F.Cu") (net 4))
 (segment (start 104.206 34.29) (end 106.172 34.29) (width 0.381) (layer "F.Cu") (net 4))
 (segment (start 85.907 55.502) (end 85.907 56.189) (width 0.381) (layer "F.Cu") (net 4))
 (segment (start 100.484 43.481) (end 98.8568 41.8538) (width 0.381) (layer "F.Cu") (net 7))
 (segment (start 98.8568 41.8538) (end 98.8568 37.0992) (width 0.381) (layer "F.Cu") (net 7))
 (segment (start 98.8568 37.0992) (end 99.871 36.085) (width 0.381) (layer "F.Cu") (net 7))
 (segment (start 96.52 42.495) (end 96.52 36.896) (width 0.381) (layer "F.Cu") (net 6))
 (segment (start 96.52 36.896) (end 97.331 36.085) (width 0.381) (layer "F.Cu") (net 6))
 (segment (start 94.772 43.481) (end 95.534 43.481) (width 0.381) (layer "F.Cu") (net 6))
 (segment (start 95.534 43.481) (end 96.52 42.495) (width 0.381) (layer "F.Cu") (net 6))
 (segment (start 109.365 57.347) (end 108.068 57.347) (width 0.508) (layer "F.Cu") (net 3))
 (segment (start 114.677 59.445) (end 112.579 57.347) (width 0.508) (layer "F.Cu") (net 3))
 (segment (start 108.068 57.347) (end 104.938 60.477) (width 0.508) (layer "F.Cu") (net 3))
 (segment (start 112.579 57.347) (end 109.365 57.347) (width 0.508) (layer "F.Cu") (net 3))
 (segment (start 101.458999 46.021) (end 104.938 49.500001) (width 0.381) (layer "F.Cu") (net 11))
 (segment (start 100.484 46.021) (end 101.458999 46.021) (width 0.381) (layer "F.Cu") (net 11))
 (segment (start 104.938 49.500001) (end 104.938 50.317) (width 0.381) (layer "F.Cu") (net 11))
 (segment (start 102.155 44.751) (end 103.163 45.759) (width 0.381) (layer "F.Cu") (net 5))
 (segment (start 104.549 42.069) (end 106.485 40.133) (width 0.508) (layer "F.Cu") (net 5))
 (segment (start 103.163 45.759) (end 104.549 45.759) (width 0.381) (layer "F.Cu") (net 5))
 (segment (start 100.484 44.751) (end 102.155 44.751) (width 0.381) (layer "F.Cu") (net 5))
 (segment (start 104.549 45.759) (end 104.549 42.069) (width 0.508) (layer "F.Cu") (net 5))
 (segment (start 92.456 41.91) (end 91.44 40.894) (width 0.381) (layer "F.Cu") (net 10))
 (segment (start 91.44 40.894) (end 83.115 40.894) (width 0.381) (layer "F.Cu") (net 10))
 (segment (start 92.456 44.45) (end 92.456 41.91) (width 0.381) (layer "F.Cu") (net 10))
 (segment (start 94.027 46.021) (end 92.456 44.45) (width 0.381) (layer "F.Cu") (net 10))
 (segment (start 83.115 40.894) (end 81.062 42.947) (width 0.381) (layer "F.Cu") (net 10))
 (segment (start 95.534 46.021) (end 94.027 46.021) (width 0.381) (layer "F.Cu") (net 10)))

